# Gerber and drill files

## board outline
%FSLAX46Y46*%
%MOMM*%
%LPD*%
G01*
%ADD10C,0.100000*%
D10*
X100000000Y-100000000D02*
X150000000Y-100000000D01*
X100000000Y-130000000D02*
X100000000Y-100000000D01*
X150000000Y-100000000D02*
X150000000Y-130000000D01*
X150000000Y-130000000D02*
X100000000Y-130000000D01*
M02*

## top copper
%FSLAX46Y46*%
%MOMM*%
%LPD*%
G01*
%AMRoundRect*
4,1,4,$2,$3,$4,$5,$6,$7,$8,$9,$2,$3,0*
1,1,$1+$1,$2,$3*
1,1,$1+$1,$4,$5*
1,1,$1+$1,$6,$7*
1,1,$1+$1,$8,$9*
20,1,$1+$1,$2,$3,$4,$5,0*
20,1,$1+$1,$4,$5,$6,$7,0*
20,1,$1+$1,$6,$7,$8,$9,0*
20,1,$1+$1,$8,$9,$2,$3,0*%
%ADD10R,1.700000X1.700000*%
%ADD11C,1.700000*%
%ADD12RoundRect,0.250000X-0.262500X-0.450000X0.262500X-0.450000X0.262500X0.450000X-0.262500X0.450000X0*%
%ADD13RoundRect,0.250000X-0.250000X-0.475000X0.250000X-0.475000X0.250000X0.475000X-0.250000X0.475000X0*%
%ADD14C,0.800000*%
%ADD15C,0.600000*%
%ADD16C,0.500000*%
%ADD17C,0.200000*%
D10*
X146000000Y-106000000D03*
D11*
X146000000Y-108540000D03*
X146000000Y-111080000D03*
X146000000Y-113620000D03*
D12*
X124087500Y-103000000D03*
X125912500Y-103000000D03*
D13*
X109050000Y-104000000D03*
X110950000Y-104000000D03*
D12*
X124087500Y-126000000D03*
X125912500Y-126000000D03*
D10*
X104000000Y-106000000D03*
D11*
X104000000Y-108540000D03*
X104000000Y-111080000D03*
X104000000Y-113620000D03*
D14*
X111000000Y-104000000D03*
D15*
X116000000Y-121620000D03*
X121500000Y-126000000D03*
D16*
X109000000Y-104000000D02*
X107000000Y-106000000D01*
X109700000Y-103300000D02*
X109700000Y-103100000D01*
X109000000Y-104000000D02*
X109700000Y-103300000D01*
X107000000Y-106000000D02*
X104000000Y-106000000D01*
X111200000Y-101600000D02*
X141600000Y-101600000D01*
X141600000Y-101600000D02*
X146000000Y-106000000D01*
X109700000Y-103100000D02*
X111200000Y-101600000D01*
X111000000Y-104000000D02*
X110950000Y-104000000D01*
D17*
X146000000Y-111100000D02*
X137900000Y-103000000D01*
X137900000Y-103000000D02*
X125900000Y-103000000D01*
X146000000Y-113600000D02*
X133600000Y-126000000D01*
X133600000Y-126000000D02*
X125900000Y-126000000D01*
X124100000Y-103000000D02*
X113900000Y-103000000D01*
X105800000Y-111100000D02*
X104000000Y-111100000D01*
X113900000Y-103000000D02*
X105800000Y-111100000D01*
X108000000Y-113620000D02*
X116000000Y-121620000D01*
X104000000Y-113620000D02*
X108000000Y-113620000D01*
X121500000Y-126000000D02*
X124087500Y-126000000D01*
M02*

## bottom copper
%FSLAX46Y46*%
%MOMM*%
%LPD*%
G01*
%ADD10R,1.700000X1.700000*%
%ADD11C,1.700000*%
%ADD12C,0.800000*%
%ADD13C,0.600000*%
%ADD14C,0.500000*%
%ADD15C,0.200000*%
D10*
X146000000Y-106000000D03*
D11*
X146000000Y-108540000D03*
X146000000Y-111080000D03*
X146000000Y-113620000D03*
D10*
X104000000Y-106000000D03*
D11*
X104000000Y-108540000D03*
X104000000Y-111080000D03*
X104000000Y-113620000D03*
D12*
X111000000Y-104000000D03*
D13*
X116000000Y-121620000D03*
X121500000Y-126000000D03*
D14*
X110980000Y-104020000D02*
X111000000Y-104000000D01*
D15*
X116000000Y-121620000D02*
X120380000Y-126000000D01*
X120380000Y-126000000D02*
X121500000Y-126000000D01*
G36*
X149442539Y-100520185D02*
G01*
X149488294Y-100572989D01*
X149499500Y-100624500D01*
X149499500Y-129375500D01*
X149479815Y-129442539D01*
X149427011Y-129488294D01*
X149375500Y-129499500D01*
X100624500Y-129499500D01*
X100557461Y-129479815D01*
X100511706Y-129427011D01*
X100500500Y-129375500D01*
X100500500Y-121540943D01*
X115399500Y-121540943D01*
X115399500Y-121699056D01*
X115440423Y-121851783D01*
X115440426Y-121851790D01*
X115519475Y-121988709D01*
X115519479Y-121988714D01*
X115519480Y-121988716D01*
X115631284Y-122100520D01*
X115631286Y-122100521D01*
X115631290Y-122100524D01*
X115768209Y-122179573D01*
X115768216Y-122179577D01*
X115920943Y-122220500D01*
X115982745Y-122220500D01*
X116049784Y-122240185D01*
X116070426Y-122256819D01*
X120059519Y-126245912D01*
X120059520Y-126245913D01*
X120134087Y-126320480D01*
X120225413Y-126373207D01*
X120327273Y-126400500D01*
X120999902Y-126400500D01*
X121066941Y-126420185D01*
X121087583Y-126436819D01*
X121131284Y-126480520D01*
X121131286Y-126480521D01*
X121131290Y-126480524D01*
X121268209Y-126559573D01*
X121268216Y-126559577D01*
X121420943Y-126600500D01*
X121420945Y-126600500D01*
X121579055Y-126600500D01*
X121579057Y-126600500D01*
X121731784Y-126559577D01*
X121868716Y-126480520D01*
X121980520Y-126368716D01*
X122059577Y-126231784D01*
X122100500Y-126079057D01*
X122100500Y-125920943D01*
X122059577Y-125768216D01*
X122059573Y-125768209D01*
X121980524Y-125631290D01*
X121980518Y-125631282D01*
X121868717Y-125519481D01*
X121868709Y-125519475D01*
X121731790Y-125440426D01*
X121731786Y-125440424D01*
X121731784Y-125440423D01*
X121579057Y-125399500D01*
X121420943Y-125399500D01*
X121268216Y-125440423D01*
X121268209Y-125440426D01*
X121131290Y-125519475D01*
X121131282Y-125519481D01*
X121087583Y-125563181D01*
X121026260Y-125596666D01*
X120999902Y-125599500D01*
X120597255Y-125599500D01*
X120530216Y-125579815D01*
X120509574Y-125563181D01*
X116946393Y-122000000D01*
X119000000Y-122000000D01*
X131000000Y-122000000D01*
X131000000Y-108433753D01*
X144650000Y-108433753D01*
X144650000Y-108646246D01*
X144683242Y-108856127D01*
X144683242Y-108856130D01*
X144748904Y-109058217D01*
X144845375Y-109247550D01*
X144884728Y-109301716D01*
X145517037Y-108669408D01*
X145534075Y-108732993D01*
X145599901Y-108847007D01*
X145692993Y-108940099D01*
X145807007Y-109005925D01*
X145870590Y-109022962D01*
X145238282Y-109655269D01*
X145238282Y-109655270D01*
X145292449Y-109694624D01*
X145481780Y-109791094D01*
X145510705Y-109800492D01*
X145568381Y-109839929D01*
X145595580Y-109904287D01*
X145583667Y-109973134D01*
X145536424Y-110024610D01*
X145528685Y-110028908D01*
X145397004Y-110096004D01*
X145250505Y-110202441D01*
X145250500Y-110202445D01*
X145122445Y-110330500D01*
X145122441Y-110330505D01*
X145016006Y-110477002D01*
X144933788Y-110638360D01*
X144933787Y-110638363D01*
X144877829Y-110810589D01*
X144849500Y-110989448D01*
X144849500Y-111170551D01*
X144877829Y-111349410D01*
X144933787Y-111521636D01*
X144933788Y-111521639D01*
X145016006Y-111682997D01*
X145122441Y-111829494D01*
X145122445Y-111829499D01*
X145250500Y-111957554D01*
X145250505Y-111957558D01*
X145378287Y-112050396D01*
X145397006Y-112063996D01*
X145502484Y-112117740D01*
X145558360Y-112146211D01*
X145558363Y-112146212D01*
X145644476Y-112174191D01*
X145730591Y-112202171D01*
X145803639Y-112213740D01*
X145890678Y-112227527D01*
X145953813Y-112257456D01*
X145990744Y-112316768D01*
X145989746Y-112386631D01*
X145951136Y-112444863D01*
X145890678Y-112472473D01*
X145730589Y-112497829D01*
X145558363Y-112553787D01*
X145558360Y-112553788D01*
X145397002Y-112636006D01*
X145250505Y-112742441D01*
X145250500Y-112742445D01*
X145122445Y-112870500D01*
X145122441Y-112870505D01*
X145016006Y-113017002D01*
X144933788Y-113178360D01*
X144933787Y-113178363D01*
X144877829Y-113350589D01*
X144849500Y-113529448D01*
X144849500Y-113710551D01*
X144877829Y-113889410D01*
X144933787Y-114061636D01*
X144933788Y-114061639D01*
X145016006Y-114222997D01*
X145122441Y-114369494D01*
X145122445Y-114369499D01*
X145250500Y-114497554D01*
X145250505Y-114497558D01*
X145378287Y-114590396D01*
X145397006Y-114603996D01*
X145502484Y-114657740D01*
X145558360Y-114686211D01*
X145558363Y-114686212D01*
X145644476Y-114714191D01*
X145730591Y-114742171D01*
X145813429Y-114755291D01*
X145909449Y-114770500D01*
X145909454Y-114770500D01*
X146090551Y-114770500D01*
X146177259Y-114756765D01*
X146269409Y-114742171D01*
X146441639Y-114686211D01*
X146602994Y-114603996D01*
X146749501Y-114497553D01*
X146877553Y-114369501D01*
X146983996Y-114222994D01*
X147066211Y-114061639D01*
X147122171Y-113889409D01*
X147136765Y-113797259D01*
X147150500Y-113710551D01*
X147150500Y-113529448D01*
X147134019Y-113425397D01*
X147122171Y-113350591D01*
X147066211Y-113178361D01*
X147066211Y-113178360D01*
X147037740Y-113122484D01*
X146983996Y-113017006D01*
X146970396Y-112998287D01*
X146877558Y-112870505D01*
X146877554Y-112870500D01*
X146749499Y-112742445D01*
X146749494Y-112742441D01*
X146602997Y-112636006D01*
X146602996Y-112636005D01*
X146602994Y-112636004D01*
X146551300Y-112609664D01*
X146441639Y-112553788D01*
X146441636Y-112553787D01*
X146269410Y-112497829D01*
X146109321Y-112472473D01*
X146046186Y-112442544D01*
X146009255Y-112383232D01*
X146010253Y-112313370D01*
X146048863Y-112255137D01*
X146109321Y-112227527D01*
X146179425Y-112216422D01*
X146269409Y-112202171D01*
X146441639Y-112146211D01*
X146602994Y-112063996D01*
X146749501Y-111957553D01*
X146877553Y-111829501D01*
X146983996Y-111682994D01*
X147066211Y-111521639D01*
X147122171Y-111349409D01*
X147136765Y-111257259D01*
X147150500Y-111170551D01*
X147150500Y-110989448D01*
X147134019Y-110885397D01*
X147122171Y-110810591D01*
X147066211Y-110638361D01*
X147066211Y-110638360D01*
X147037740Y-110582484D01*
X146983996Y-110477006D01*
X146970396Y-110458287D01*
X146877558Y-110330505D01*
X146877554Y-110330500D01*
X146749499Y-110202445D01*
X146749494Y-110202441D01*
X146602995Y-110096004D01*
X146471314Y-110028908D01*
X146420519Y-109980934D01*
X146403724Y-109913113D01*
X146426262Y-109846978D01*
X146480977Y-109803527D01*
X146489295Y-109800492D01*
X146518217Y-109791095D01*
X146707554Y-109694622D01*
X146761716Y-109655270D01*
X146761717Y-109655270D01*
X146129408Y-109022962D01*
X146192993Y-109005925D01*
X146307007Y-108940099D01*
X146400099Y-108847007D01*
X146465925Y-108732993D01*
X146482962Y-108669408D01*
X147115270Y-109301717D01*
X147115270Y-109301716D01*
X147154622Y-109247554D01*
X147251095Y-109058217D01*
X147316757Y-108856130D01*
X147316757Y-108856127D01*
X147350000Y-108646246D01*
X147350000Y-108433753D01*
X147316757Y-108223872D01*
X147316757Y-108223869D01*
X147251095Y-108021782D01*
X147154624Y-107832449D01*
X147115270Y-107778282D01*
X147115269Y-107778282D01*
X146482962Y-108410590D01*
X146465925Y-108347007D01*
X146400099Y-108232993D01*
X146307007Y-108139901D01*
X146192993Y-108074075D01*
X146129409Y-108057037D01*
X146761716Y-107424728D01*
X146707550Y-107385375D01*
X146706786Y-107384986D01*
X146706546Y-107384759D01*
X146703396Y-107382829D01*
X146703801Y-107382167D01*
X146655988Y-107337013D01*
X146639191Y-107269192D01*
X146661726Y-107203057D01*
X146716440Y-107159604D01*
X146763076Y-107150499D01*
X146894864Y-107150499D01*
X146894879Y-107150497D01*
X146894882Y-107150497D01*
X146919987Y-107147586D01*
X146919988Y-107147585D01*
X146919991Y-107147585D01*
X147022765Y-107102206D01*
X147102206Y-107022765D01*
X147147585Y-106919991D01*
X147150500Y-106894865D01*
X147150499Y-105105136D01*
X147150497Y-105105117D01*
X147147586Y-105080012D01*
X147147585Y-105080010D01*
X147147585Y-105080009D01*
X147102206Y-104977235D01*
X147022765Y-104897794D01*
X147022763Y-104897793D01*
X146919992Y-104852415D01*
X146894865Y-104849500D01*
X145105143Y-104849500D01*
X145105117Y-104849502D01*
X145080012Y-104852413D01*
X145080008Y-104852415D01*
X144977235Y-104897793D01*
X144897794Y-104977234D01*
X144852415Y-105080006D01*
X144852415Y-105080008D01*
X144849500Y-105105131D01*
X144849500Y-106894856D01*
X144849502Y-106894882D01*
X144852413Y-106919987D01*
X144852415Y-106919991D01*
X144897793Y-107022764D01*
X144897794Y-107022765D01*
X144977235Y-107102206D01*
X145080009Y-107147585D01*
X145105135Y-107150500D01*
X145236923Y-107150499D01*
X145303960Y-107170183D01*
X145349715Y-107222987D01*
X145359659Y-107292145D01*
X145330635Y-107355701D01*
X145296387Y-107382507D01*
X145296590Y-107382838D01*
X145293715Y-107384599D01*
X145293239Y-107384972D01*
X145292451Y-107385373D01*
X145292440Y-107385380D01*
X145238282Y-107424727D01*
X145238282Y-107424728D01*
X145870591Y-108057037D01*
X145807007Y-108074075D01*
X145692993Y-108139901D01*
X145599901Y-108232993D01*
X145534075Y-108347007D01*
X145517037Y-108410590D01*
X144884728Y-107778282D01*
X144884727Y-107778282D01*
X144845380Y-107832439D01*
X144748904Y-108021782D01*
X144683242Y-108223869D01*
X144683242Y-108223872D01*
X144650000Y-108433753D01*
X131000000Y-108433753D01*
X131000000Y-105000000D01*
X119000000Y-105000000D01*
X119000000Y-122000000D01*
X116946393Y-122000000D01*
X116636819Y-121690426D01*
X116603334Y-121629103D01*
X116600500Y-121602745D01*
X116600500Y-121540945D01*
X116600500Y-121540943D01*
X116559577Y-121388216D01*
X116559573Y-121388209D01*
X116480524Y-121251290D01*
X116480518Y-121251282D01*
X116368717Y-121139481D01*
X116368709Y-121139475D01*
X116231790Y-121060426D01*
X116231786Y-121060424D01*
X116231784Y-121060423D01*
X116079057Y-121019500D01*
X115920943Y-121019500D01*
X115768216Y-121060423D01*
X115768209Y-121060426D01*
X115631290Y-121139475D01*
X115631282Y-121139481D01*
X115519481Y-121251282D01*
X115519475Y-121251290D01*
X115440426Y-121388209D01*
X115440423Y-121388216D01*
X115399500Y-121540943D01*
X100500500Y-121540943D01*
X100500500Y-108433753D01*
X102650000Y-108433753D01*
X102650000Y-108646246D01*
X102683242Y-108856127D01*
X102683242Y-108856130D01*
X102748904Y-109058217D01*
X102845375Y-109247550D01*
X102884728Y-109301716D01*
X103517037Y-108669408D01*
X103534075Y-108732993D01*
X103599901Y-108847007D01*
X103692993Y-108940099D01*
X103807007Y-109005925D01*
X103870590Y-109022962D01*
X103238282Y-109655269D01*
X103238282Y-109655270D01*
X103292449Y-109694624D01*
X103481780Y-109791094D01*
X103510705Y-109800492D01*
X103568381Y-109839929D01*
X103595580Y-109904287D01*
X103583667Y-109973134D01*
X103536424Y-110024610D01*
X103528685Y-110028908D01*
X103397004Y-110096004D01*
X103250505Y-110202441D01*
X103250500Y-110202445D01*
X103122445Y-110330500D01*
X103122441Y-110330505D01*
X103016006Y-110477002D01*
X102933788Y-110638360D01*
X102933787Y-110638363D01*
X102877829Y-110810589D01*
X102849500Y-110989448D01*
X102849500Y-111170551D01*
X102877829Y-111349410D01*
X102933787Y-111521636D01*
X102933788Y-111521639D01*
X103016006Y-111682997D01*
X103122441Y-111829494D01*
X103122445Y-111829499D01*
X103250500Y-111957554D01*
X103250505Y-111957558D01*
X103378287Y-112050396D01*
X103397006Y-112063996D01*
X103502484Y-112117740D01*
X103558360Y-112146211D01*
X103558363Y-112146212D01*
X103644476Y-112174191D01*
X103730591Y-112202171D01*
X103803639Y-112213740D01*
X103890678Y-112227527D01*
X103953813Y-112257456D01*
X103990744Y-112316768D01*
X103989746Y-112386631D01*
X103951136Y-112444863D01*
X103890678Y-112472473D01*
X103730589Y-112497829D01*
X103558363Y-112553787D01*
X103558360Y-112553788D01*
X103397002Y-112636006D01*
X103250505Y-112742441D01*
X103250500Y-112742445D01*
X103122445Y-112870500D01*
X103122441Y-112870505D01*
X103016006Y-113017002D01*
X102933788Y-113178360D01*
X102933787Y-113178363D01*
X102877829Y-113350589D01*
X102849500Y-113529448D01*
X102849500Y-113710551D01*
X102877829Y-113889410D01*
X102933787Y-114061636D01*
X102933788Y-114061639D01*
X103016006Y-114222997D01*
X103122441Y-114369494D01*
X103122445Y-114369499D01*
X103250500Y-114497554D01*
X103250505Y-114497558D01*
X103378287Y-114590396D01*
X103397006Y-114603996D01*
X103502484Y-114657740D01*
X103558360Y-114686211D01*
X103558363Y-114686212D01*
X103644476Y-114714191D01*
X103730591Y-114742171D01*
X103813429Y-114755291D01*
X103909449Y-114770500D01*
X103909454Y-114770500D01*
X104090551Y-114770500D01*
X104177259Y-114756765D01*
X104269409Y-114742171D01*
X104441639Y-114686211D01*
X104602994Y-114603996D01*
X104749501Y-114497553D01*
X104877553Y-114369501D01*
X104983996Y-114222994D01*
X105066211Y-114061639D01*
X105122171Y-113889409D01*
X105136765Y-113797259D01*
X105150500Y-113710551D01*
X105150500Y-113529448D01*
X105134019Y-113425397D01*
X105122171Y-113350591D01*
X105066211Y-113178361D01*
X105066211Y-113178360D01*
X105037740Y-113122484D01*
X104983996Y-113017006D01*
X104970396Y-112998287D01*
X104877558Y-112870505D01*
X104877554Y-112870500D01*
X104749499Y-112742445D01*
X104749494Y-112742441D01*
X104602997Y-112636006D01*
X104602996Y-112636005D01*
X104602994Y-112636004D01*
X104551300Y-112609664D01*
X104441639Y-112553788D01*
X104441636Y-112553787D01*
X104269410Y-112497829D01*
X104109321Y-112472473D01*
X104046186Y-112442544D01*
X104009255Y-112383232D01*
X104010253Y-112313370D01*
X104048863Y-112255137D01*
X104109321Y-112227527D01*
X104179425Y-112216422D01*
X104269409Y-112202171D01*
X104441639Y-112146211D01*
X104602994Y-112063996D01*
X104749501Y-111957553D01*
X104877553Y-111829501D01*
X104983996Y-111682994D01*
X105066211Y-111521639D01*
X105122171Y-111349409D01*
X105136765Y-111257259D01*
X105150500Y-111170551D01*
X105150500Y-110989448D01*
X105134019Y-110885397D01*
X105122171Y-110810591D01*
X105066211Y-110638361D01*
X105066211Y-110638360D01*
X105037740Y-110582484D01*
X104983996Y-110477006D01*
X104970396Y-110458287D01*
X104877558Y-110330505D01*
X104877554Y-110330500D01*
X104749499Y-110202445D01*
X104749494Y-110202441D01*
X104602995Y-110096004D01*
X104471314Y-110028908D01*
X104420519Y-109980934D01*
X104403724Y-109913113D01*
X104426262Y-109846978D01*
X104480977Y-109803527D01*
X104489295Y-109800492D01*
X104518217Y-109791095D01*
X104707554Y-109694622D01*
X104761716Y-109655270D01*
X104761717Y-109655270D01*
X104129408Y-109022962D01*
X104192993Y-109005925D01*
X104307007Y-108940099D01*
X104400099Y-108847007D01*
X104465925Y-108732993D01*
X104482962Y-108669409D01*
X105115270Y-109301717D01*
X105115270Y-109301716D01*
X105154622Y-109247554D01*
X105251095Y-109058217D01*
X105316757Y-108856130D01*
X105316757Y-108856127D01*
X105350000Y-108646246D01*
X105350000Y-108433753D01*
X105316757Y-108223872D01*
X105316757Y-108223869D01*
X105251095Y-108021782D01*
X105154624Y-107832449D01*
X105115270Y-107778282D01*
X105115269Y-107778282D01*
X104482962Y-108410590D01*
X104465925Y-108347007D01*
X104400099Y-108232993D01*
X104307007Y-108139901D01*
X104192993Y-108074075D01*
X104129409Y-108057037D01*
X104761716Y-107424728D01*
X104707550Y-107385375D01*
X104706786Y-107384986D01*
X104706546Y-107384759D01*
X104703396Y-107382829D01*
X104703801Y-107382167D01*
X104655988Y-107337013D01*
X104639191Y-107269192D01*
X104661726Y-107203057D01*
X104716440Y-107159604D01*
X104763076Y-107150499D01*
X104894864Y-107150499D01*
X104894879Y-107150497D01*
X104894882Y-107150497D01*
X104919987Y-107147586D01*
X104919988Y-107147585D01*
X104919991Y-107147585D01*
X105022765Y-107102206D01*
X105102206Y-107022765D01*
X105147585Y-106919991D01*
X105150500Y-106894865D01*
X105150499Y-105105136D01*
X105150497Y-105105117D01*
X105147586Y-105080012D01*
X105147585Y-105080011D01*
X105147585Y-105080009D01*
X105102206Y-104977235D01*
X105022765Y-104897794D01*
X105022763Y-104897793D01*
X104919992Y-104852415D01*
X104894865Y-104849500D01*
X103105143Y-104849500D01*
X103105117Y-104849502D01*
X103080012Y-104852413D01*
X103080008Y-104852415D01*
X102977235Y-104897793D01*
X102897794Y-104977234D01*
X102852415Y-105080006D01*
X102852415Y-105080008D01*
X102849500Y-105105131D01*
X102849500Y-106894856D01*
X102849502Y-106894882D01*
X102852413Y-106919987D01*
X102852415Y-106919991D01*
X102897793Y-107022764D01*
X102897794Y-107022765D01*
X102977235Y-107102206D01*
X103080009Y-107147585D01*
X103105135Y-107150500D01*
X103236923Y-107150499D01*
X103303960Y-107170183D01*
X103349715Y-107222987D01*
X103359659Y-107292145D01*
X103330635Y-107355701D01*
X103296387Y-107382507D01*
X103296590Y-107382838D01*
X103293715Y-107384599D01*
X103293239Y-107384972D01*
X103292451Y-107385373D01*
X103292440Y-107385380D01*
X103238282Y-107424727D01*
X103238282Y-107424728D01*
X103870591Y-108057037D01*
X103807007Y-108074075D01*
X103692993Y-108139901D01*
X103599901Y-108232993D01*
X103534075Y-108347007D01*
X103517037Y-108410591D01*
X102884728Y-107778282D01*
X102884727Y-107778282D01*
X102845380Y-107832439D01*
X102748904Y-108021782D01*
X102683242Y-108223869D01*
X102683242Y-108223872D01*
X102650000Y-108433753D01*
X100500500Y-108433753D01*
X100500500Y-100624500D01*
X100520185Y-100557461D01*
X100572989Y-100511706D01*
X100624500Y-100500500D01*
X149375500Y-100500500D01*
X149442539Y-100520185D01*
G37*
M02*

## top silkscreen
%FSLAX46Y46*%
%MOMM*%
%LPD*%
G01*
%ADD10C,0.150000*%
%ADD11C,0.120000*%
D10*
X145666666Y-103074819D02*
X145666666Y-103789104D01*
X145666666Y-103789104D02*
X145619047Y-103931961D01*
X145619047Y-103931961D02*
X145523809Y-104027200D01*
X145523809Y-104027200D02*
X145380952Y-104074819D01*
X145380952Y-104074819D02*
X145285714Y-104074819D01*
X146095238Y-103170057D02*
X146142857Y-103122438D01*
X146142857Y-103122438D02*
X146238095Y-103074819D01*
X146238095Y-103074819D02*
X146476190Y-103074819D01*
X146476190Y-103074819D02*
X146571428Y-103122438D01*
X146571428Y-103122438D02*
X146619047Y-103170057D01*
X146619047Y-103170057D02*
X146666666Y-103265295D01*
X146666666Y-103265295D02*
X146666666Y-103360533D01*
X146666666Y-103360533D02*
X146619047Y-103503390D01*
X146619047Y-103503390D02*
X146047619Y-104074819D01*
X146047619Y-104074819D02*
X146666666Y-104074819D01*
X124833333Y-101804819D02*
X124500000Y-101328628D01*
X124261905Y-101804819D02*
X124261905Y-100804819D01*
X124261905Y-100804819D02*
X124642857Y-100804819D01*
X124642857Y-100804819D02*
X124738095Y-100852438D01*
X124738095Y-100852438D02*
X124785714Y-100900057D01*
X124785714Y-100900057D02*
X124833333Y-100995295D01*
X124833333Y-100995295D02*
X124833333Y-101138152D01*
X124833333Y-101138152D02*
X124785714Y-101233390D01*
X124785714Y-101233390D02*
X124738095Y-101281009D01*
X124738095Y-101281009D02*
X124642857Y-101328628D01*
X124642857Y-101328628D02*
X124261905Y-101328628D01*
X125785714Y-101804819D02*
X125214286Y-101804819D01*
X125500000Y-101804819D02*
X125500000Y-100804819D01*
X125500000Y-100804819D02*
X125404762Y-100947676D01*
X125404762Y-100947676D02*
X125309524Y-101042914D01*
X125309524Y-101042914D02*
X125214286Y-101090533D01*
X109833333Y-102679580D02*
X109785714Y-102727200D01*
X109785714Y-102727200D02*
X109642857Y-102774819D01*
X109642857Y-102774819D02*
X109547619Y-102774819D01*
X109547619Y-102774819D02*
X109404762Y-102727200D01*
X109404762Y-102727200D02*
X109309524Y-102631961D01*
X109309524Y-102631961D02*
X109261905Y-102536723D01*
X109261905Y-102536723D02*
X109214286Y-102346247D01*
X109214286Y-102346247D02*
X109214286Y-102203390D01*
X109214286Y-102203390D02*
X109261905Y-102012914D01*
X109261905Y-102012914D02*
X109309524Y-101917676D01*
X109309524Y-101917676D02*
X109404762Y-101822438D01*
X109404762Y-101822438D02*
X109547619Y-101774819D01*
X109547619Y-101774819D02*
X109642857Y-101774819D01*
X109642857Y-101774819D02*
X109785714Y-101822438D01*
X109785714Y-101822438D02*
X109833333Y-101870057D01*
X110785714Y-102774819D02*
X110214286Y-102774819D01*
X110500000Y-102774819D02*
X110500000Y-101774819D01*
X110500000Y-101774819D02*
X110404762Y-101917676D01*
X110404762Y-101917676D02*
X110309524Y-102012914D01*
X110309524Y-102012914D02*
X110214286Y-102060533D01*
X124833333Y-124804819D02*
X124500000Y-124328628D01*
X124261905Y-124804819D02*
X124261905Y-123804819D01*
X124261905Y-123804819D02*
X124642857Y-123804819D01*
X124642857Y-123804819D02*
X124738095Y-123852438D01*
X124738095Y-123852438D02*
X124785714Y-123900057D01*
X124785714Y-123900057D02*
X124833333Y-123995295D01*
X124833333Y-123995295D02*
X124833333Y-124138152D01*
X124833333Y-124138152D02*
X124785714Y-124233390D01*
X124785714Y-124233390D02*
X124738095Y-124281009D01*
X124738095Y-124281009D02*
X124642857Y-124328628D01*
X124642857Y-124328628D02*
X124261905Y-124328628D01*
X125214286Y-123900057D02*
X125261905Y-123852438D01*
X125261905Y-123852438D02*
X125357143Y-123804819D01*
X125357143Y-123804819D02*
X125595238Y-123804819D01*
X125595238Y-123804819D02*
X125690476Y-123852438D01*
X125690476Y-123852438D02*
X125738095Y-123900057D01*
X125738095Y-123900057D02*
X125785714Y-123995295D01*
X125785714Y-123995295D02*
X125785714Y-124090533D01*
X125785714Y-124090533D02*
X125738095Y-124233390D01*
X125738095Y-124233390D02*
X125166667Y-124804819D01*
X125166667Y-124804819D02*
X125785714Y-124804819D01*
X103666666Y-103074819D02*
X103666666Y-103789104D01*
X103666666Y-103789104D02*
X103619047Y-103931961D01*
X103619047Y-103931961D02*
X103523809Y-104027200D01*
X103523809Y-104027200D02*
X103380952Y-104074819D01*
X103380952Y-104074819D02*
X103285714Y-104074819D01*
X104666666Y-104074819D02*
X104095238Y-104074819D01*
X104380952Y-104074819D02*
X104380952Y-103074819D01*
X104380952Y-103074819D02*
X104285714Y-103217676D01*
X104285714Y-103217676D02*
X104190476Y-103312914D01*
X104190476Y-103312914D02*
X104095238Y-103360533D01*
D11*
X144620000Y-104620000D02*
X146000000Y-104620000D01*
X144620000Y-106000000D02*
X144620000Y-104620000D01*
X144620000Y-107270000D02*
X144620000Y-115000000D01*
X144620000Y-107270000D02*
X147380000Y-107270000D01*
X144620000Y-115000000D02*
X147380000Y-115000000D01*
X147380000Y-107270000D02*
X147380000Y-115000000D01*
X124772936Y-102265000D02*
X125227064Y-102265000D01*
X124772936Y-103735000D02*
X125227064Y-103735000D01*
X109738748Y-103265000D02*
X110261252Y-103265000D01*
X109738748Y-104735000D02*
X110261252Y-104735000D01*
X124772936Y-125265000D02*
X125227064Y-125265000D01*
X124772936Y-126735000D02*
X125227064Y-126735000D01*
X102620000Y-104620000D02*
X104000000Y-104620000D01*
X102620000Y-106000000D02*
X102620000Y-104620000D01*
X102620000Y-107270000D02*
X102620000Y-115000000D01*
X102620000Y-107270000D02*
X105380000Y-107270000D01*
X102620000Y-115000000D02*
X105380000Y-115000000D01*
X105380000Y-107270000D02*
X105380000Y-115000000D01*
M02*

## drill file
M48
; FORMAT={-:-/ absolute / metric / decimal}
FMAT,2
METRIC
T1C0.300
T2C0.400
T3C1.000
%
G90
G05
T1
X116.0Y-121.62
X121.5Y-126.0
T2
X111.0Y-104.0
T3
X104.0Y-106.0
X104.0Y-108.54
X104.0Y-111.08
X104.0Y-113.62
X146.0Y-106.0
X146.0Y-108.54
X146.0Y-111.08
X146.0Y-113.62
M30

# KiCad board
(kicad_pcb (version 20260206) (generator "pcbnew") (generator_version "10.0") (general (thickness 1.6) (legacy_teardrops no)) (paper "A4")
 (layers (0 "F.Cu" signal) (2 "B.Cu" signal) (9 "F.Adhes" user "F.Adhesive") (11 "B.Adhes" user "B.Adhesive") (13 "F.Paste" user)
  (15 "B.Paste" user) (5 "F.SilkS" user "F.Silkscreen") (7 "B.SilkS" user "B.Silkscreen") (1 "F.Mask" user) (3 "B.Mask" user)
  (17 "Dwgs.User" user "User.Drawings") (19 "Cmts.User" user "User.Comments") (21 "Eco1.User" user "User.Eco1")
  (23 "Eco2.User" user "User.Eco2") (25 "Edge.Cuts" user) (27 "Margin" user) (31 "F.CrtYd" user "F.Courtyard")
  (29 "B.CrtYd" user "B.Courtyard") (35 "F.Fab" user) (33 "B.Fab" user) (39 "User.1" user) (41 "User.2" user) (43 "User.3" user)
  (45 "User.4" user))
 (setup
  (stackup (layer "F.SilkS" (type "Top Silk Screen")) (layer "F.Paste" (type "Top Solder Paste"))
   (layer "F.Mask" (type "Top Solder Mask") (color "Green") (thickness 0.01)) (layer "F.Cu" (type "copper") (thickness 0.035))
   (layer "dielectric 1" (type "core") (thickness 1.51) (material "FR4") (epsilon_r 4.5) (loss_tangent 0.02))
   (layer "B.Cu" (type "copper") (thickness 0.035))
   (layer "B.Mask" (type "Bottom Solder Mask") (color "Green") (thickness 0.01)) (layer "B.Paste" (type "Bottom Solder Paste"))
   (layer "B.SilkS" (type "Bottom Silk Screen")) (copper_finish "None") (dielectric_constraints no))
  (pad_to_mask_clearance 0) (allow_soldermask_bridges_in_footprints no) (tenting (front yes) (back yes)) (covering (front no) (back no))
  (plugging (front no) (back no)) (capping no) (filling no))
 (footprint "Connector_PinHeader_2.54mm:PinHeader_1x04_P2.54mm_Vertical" (layer "F.Cu") (at 146 106)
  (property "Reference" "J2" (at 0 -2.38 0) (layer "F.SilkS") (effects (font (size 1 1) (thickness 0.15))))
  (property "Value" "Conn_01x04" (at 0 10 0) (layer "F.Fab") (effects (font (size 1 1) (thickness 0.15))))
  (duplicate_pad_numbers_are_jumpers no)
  (fp_line (start -1.38 -1.38) (end 0 -1.38) (stroke (width 0.12) (type solid)) (layer "F.SilkS"))
  (fp_line (start -1.38 0) (end -1.38 -1.38) (stroke (width 0.12) (type solid)) (layer "F.SilkS"))
  (fp_line (start -1.38 1.27) (end -1.38 9) (stroke (width 0.12) (type solid)) (layer "F.SilkS"))
  (fp_line (start -1.38 1.27) (end 1.38 1.27) (stroke (width 0.12) (type solid)) (layer "F.SilkS"))
  (fp_line (start -1.38 9) (end 1.38 9) (stroke (width 0.12) (type solid)) (layer "F.SilkS"))
  (fp_line (start 1.38 1.27) (end 1.38 9) (stroke (width 0.12) (type solid)) (layer "F.SilkS"))
  (pad "1" thru_hole rect (at 0 0) (size 1.7 1.7) (drill 1) (layers "*.Cu" "*.Mask") (remove_unused_layers no) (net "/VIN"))
  (pad "2" thru_hole circle (at 0 2.54) (size 1.7 1.7) (drill 1) (layers "*.Cu" "*.Mask") (remove_unused_layers no) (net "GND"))
  (pad "3" thru_hole circle (at 0 5.08) (size 1.7 1.7) (drill 1) (layers "*.Cu" "*.Mask") (remove_unused_layers no) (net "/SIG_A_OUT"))
  (pad "4" thru_hole circle (at 0 7.62) (size 1.7 1.7) (drill 1) (layers "*.Cu" "*.Mask") (remove_unused_layers no) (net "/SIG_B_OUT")))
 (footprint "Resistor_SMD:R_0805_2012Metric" (layer "F.Cu") (at 125 103)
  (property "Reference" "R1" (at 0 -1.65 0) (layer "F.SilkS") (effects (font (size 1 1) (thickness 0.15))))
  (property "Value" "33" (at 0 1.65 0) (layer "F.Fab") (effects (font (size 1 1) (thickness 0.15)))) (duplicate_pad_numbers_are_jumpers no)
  (fp_line (start -0.227064 -0.735) (end 0.227064 -0.735) (stroke (width 0.12) (type solid)) (layer "F.SilkS"))
  (fp_line (start -0.227064 0.735) (end 0.227064 0.735) (stroke (width 0.12) (type solid)) (layer "F.SilkS"))
  (pad "1" smd roundrect (at -0.9125 0) (size 1.025 1.4) (layers "F.Cu" "F.Mask" "F.Paste") (roundrect_rratio 0.243902) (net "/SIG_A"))
  (pad "2" smd roundrect (at 0.9125 0) (size 1.025 1.4) (layers "F.Cu" "F.Mask" "F.Paste") (roundrect_rratio 0.243902) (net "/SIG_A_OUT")))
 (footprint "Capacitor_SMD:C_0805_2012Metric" (layer "F.Cu") (at 110 104)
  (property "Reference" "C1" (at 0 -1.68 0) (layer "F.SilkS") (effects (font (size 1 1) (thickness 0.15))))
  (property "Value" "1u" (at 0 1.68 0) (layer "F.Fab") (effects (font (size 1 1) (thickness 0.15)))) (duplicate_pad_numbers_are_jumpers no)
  (fp_line (start -0.261252 -0.735) (end 0.261252 -0.735) (stroke (width 0.12) (type solid)) (layer "F.SilkS"))
  (fp_line (start -0.261252 0.735) (end 0.261252 0.735) (stroke (width 0.12) (type solid)) (layer "F.SilkS"))
  (pad "1" smd roundrect (at -0.95 0) (size 1 1.45) (layers "F.Cu" "F.Mask" "F.Paste") (roundrect_rratio 0.25) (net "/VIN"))
  (pad "2" smd roundrect (at 0.95 0) (size 1 1.45) (layers "F.Cu" "F.Mask" "F.Paste") (roundrect_rratio 0.25) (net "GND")))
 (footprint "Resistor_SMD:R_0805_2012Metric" (layer "F.Cu") (at 125 126)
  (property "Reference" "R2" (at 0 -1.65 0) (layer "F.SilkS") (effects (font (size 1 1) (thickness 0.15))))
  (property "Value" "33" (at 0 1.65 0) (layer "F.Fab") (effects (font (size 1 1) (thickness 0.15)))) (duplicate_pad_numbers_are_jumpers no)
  (fp_line (start -0.227064 -0.735) (end 0.227064 -0.735) (stroke (width 0.12) (type solid)) (layer "F.SilkS"))
  (fp_line (start -0.227064 0.735) (end 0.227064 0.735) (stroke (width 0.12) (type solid)) (layer "F.SilkS"))
  (pad "1" smd roundrect (at -0.9125 0) (size 1.025 1.4) (layers "F.Cu" "F.Mask" "F.Paste") (roundrect_rratio 0.243902) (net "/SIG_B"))
  (pad "2" smd roundrect (at 0.9125 0) (size 1.025 1.4) (layers "F.Cu" "F.Mask" "F.Paste") (roundrect_rratio 0.243902) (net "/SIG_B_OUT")))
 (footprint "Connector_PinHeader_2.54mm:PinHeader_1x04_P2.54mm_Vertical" (layer "F.Cu") (at 104 106)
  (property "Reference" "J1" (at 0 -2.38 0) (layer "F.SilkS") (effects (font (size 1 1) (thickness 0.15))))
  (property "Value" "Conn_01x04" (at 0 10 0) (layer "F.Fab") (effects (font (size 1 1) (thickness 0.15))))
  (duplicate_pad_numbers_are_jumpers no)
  (fp_line (start -1.38 -1.38) (end 0 -1.38) (stroke (width 0.12) (type solid)) (layer "F.SilkS"))
  (fp_line (start -1.38 0) (end -1.38 -1.38) (stroke (width 0.12) (type solid)) (layer "F.SilkS"))
  (fp_line (start -1.38 1.27) (end -1.38 9) (stroke (width 0.12) (type solid)) (layer "F.SilkS"))
  (fp_line (start -1.38 1.27) (end 1.38 1.27) (stroke (width 0.12) (type solid)) (layer "F.SilkS"))
  (fp_line (start -1.38 9) (end 1.38 9) (stroke (width 0.12) (type solid)) (layer "F.SilkS"))
  (fp_line (start 1.38 1.27) (end 1.38 9) (stroke (width 0.12) (type solid)) (layer "F.SilkS"))
  (pad "1" thru_hole rect (at 0 0) (size 1.7 1.7) (drill 1) (layers "*.Cu" "*.Mask") (remove_unused_layers no) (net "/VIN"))
  (pad "2" thru_hole circle (at 0 2.54) (size 1.7 1.7) (drill 1) (layers "*.Cu" "*.Mask") (remove_unused_layers no) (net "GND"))
  (pad "3" thru_hole circle (at 0 5.08) (size 1.7 1.7) (drill 1) (layers "*.Cu" "*.Mask") (remove_unused_layers no) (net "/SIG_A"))
  (pad "4" thru_hole circle (at 0 7.62) (size 1.7 1.7) (drill 1) (layers "*.Cu" "*.Mask") (remove_unused_layers no) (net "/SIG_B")))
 (gr_line (start 100 100) (end 150 100) (stroke (width 0.1) (type default)) (layer "Edge.Cuts"))
 (gr_line (start 100 130) (end 100 100) (stroke (width 0.1) (type default)) (layer "Edge.Cuts"))
 (gr_line (start 150 100) (end 150 130) (stroke (width 0.1) (type default)) (layer "Edge.Cuts"))
 (gr_line (start 150 130) (end 100 130) (stroke (width 0.1) (type default)) (layer "Edge.Cuts"))
 (segment (start 109 104) (end 107 106) (width 0.5) (layer "F.Cu") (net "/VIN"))
 (segment (start 109.7 103.3) (end 109.7 103.1) (width 0.5) (layer "F.Cu") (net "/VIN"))
 (segment (start 109 104) (end 109.7 103.3) (width 0.5) (layer "F.Cu") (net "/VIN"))
 (segment (start 107 106) (end 104 106) (width 0.5) (layer "F.Cu") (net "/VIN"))
 (segment (start 111.2 101.6) (end 141.6 101.6) (width 0.5) (layer "F.Cu") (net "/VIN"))
 (segment (start 141.6 101.6) (end 146 106) (width 0.5) (layer "F.Cu") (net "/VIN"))
 (segment (start 109.7 103.1) (end 111.2 101.6) (width 0.5) (layer "F.Cu") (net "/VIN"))
 (segment (start 111 104) (end 110.95 104) (width 0.5) (layer "F.Cu") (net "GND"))
 (via (at 111 104) (size 0.8) (drill 0.4) (layers "F.Cu" "B.Cu") (capping yes) (filling yes) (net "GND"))
 (segment (start 110.98 104.02) (end 111 104) (width 0.5) (layer "B.Cu") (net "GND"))
 (segment (start 146 111.1) (end 137.9 103) (width 0.2) (layer "F.Cu") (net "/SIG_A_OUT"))
 (segment (start 137.9 103) (end 125.9 103) (width 0.2) (layer "F.Cu") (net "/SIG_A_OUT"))
 (segment (start 146 113.6) (end 133.6 126) (width 0.2) (layer "F.Cu") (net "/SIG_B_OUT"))
 (segment (start 133.6 126) (end 125.9 126) (width 0.2) (layer "F.Cu") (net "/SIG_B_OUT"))
 (segment (start 124.1 103) (end 113.9 103) (width 0.2) (layer "F.Cu") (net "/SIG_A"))
 (segment (start 105.8 111.1) (end 104 111.1) (width 0.2) (layer "F.Cu") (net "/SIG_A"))
 (segment (start 113.9 103) (end 105.8 111.1) (width 0.2) (layer "F.Cu") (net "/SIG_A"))
 (segment (start 108 113.62) (end 116 121.62) (width 0.2) (locked yes) (layer "F.Cu") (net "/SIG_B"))
 (segment (start 104 113.62) (end 108 113.62) (width 0.2) (locked yes) (layer "F.Cu") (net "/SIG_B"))
 (segment (start 121.5 126) (end 124.0875 126) (width 0.2) (locked yes) (layer "F.Cu") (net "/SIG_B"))
 (via (at 116 121.62) (size 0.6) (drill 0.3) (layers "F.Cu" "B.Cu") (locked yes) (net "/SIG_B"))
 (via (at 121.5 126) (size 0.6) (drill 0.3) (layers "F.Cu" "B.Cu") (locked yes) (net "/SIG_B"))
 (segment (start 116 121.62) (end 120.38 126) (width 0.2) (locked yes) (layer "B.Cu") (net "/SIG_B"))
 (segment (start 120.38 126) (end 121.5 126) (width 0.2) (locked yes) (layer "B.Cu") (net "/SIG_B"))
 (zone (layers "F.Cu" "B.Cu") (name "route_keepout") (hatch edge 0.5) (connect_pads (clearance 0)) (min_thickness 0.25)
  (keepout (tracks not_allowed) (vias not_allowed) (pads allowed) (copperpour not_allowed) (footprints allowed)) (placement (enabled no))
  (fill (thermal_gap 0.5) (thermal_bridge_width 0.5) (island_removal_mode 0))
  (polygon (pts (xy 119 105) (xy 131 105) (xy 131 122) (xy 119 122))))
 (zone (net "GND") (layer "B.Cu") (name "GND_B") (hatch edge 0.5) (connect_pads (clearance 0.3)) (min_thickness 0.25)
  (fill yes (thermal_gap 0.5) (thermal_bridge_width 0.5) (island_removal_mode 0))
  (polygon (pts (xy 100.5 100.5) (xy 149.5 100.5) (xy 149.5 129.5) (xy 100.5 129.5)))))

